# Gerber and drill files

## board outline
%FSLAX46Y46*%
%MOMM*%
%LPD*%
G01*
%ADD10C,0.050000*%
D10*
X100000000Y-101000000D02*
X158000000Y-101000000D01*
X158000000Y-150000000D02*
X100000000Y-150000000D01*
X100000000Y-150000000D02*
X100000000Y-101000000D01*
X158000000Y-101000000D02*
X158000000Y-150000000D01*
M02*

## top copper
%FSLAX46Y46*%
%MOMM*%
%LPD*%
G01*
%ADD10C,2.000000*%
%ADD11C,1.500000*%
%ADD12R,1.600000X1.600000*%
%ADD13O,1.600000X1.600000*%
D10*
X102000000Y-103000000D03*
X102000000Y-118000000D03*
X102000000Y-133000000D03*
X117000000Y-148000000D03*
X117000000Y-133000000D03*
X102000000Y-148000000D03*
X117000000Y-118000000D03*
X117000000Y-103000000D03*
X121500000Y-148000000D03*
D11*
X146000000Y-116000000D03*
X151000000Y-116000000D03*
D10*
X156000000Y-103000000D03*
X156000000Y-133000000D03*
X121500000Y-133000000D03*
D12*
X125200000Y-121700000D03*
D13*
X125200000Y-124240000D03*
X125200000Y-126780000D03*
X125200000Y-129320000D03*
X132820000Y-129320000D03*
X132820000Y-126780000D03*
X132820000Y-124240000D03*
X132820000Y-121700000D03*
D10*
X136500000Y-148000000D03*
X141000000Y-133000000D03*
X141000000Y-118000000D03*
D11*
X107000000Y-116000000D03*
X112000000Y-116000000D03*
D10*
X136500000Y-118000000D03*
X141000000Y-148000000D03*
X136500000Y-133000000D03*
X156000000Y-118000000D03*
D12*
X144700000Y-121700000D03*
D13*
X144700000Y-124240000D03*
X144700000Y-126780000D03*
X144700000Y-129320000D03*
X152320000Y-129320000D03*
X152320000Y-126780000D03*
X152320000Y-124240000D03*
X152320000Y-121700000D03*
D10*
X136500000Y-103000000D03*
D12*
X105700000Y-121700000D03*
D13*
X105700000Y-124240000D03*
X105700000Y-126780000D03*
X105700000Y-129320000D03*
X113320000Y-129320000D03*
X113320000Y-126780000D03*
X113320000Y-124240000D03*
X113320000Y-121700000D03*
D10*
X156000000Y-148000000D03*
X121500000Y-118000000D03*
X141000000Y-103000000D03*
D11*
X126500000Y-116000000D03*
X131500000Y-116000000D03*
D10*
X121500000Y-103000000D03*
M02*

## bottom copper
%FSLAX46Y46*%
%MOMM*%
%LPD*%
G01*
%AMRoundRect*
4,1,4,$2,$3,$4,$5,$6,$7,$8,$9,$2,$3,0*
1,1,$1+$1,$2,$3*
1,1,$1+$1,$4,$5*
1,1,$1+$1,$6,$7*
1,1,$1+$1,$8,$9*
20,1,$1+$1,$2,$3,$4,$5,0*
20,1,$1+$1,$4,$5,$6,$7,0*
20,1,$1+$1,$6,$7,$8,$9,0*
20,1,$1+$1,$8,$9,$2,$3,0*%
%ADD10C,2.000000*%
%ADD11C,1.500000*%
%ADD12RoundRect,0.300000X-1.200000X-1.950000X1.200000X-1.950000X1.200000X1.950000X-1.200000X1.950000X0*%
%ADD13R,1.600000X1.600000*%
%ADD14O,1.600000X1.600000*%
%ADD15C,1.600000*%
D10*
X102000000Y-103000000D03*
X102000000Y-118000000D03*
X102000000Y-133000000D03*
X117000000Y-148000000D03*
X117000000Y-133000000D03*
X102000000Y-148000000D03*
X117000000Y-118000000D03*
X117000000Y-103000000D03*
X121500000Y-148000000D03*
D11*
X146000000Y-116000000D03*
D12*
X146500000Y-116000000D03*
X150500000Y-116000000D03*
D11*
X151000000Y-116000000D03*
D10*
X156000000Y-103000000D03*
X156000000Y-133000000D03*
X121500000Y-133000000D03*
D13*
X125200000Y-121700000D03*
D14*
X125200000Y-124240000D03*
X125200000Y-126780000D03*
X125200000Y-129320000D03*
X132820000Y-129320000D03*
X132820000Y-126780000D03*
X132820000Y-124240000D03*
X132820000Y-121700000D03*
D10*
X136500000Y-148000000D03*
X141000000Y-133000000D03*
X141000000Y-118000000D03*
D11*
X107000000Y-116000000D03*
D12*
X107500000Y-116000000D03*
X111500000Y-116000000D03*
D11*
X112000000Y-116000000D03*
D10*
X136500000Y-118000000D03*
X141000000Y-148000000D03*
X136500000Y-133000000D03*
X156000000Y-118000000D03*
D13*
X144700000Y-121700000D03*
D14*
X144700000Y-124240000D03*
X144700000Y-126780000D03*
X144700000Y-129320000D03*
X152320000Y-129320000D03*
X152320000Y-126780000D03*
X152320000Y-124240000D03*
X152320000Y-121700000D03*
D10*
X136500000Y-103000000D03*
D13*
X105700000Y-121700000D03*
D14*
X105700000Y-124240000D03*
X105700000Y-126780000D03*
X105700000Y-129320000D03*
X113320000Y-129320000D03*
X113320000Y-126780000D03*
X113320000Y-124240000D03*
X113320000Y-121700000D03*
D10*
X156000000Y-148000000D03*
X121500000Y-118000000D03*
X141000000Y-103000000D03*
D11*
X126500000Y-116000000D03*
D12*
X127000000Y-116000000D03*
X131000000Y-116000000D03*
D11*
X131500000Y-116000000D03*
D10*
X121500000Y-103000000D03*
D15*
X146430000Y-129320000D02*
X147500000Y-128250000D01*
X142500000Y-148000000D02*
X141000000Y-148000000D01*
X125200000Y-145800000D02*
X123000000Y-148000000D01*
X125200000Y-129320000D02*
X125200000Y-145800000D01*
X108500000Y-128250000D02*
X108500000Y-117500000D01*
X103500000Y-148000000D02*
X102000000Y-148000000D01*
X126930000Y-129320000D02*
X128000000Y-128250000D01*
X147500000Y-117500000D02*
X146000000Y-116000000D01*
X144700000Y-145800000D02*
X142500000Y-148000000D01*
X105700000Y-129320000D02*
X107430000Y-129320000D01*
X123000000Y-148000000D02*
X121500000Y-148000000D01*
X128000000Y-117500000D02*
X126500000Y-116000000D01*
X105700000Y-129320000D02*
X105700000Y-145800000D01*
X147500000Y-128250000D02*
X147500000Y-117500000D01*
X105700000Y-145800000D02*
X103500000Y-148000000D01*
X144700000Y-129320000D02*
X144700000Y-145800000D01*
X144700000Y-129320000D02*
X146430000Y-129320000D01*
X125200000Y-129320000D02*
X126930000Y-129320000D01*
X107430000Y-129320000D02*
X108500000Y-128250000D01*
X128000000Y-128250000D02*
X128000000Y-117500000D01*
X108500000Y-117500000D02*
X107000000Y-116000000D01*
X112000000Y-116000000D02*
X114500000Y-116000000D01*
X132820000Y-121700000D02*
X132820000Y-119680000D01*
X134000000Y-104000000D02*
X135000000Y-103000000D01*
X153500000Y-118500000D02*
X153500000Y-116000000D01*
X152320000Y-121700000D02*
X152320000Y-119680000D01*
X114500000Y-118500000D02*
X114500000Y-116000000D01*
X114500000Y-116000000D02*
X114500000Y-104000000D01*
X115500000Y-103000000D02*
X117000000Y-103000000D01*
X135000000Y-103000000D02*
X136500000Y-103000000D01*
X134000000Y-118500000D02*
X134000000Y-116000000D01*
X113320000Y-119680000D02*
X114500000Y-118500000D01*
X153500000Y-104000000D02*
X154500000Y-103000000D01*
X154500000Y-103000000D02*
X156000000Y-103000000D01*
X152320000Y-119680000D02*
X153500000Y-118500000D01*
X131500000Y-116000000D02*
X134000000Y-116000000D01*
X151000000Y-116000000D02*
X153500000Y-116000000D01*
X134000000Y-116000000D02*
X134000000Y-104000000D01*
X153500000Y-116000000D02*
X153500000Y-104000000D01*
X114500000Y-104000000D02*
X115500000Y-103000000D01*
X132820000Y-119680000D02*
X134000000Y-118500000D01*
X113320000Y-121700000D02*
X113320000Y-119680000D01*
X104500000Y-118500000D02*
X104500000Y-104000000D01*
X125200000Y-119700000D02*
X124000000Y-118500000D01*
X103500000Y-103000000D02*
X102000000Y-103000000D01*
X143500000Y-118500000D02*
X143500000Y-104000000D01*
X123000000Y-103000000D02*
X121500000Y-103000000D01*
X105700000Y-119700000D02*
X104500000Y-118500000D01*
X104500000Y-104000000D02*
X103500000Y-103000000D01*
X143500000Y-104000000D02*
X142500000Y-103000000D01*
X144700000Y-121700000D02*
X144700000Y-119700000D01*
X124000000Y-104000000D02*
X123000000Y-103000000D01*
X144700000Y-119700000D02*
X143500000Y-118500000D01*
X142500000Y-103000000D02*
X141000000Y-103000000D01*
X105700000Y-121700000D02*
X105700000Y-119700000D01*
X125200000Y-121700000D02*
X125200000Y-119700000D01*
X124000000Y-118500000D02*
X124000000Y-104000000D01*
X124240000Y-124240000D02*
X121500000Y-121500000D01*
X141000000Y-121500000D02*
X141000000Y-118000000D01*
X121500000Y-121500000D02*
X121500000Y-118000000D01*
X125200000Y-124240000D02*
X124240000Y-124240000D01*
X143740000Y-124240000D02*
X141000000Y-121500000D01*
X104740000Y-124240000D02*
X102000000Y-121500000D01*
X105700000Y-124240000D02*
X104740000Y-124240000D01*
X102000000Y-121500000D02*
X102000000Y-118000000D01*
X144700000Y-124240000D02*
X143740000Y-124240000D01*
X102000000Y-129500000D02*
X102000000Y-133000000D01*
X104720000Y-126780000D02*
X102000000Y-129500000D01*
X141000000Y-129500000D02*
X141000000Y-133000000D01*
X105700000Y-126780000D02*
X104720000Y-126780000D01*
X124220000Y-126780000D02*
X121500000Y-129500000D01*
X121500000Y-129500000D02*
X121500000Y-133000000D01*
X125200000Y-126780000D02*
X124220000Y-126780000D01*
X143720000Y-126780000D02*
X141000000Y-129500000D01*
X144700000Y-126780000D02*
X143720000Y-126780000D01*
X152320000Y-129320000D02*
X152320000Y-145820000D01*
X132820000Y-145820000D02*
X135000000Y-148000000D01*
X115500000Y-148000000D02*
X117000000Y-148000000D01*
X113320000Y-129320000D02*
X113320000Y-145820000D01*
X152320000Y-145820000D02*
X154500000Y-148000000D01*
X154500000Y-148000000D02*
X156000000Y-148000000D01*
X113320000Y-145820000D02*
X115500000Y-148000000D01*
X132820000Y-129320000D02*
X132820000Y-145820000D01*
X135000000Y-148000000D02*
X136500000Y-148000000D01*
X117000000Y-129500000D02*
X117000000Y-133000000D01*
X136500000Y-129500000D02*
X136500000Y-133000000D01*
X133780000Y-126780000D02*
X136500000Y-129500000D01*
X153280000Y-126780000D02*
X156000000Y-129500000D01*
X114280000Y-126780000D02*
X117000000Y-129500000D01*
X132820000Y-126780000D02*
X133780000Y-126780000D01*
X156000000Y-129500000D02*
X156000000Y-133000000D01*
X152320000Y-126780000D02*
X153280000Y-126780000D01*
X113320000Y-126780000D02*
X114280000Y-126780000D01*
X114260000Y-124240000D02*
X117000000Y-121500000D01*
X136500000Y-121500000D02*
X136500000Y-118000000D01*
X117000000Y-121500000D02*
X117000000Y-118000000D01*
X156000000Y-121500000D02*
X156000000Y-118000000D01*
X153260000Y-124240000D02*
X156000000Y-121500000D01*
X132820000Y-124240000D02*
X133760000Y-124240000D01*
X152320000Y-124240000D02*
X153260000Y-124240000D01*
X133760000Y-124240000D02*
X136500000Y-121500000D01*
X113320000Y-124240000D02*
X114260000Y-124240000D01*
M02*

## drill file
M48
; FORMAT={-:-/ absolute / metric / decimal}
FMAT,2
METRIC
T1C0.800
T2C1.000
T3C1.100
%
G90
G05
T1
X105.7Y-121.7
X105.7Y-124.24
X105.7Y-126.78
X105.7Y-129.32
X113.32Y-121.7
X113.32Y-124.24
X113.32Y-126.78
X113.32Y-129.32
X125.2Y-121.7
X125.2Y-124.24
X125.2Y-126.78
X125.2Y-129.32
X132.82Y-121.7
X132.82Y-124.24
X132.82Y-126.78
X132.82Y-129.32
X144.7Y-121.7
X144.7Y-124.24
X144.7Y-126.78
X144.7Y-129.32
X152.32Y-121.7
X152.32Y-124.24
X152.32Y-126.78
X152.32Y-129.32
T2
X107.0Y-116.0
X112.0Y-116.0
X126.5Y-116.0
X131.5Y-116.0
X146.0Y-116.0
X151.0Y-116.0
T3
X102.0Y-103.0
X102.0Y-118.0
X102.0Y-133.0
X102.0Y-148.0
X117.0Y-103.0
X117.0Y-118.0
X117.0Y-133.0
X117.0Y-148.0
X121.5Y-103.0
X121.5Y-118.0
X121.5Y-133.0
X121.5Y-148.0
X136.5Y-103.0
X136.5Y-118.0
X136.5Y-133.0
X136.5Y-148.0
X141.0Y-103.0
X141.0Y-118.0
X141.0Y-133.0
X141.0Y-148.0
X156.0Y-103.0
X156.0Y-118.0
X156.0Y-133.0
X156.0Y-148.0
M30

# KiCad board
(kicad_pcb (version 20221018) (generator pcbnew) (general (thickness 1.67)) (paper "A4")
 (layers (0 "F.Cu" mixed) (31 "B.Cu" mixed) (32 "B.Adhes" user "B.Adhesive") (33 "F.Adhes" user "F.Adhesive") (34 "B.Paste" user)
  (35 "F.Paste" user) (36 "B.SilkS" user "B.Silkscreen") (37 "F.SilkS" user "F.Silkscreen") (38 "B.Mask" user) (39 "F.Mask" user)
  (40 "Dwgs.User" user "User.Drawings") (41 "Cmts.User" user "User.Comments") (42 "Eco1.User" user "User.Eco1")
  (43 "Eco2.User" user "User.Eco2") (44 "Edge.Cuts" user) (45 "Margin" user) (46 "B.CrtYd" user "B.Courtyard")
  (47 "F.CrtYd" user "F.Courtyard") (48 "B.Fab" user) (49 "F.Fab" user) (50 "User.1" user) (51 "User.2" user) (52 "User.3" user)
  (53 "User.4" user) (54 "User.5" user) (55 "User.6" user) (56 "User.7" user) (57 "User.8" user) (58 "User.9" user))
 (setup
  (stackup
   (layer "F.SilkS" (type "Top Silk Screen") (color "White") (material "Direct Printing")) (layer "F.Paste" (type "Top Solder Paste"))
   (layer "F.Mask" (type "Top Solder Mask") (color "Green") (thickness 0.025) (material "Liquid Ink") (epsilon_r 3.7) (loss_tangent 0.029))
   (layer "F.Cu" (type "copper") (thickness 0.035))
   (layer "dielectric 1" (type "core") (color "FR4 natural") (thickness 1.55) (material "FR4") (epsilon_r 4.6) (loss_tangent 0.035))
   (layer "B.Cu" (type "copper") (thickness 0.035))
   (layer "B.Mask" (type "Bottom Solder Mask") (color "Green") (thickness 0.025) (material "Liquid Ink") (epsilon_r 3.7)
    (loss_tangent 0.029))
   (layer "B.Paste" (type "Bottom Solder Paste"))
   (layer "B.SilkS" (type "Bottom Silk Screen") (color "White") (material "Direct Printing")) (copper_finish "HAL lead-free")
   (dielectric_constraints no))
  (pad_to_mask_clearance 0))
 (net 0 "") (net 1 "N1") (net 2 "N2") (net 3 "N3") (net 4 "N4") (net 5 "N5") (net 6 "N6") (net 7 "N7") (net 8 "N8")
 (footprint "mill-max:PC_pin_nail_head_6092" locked (layer "F.Cu") (at 102 103)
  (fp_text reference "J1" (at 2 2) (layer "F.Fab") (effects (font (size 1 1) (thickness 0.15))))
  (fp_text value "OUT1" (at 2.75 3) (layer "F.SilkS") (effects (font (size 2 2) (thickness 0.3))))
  (pad "1" thru_hole circle locked (at 0 0) (size 2 2) (drill 1.1) (layers "*.Cu" "*.Mask") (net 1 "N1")))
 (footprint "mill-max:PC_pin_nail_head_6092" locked (layer "F.Cu") (at 102 118)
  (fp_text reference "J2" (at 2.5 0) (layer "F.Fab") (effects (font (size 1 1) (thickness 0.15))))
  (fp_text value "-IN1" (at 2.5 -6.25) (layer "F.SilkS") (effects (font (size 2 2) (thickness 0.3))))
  (pad "1" thru_hole circle locked (at 0 0) (size 2 2) (drill 1.1) (layers "*.Cu" "*.Mask") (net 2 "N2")))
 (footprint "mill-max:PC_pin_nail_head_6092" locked (layer "F.Cu") (at 102 133)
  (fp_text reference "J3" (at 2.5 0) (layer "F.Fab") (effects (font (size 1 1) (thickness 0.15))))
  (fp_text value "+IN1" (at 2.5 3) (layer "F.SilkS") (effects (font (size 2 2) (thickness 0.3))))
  (pad "1" thru_hole circle locked (at 0 0) (size 2 2) (drill 1.1) (layers "*.Cu" "*.Mask") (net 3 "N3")))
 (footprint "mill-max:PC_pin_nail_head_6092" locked (layer "F.Cu") (at 117 148)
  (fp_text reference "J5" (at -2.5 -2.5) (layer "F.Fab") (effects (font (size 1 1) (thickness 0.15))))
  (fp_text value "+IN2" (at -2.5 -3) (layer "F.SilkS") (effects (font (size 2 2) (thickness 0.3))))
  (pad "1" thru_hole circle locked (at 0 0) (size 2 2) (drill 1.1) (layers "*.Cu" "*.Mask") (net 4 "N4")))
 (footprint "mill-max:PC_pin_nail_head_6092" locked (layer "F.Cu") (at 117 133)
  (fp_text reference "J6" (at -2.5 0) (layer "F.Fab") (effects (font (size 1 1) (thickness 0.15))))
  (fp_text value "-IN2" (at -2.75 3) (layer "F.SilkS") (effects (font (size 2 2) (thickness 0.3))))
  (pad "1" thru_hole circle locked (at 0 0) (size 2 2) (drill 1.1) (layers "*.Cu" "*.Mask") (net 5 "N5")))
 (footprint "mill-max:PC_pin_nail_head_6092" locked (layer "F.Cu") (at 102 148)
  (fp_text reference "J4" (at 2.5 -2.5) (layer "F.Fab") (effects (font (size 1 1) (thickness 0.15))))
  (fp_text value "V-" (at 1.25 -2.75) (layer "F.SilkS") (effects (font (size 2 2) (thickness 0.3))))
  (pad "1" thru_hole circle locked (at 0 0) (size 2 2) (drill 1.1) (layers "*.Cu" "*.Mask") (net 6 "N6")))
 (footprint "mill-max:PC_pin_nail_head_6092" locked (layer "F.Cu") (at 117 118)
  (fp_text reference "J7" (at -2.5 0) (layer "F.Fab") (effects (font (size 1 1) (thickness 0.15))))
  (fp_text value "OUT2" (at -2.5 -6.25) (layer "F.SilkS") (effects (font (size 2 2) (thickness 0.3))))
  (pad "1" thru_hole circle locked (at 0 0) (size 2 2) (drill 1.1) (layers "*.Cu" "*.Mask") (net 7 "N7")))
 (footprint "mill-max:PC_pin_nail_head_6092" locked (layer "F.Cu") (at 117 103)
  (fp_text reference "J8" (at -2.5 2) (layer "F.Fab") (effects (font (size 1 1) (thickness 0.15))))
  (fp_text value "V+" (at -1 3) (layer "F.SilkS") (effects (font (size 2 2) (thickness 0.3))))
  (pad "1" thru_hole circle locked (at 0 0) (size 2 2) (drill 1.1) (layers "*.Cu" "*.Mask") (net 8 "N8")))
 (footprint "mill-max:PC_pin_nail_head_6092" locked (layer "F.Cu") (at 121.5 148)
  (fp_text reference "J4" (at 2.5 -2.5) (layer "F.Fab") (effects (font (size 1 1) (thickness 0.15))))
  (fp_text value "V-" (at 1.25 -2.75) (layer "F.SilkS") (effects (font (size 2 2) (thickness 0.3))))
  (pad "1" thru_hole circle locked (at 0 0) (size 2 2) (drill 1.1) (layers "*.Cu" "*.Mask") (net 6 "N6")))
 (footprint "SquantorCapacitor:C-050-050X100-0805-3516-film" (layer "F.Cu") (at 148.5 116)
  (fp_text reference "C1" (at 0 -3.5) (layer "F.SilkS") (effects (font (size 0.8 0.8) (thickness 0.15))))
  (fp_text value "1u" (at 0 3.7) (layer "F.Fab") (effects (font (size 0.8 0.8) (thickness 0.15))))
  (pad "1" thru_hole circle (at -2.5 0) (size 1.5 1.5) (drill 1) (layers "*.Cu" "*.Mask") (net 6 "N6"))
  (pad "1" smd roundrect (at -2 0) (size 3 4.5) (layers "B.Cu" "B.Paste" "B.Mask") (roundrect_rratio 0.1) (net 6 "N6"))
  (pad "2" smd roundrect (at 2 0) (size 3 4.5) (layers "B.Cu" "B.Paste" "B.Mask") (roundrect_rratio 0.1) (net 8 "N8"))
  (pad "2" thru_hole circle (at 2.5 0) (size 1.5 1.5) (drill 1) (layers "*.Cu" "*.Mask") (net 8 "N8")))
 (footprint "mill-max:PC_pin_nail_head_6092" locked (layer "F.Cu") (at 156 103)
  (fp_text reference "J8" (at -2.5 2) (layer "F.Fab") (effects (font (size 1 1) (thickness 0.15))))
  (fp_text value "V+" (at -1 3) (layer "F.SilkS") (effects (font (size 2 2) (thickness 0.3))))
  (pad "1" thru_hole circle locked (at 0 0) (size 2 2) (drill 1.1) (layers "*.Cu" "*.Mask") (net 8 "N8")))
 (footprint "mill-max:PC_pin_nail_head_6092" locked (layer "F.Cu") (at 156 133)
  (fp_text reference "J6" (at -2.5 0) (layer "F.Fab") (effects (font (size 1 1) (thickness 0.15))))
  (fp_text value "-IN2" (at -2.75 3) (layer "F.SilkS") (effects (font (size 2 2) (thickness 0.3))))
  (pad "1" thru_hole circle locked (at 0 0) (size 2 2) (drill 1.1) (layers "*.Cu" "*.Mask") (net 5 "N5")))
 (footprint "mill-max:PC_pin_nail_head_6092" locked (layer "F.Cu") (at 121.5 133)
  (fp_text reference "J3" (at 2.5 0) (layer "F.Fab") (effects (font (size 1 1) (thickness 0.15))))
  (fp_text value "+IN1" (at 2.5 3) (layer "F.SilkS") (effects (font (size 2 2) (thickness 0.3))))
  (pad "1" thru_hole circle locked (at 0 0) (size 2 2) (drill 1.1) (layers "*.Cu" "*.Mask") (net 3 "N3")))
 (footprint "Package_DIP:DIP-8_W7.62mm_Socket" (layer "F.Cu") (at 125.2 121.7)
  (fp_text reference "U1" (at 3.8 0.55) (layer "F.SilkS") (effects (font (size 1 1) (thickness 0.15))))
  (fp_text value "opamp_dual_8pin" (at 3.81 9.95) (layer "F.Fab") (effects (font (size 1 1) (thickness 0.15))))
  (pad "1" thru_hole rect (at 0 0) (size 1.6 1.6) (drill 0.8) (layers "*.Cu" "*.Mask") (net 1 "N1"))
  (pad "2" thru_hole oval (at 0 2.54) (size 1.6 1.6) (drill 0.8) (layers "*.Cu" "*.Mask") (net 2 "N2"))
  (pad "3" thru_hole oval (at 0 5.08) (size 1.6 1.6) (drill 0.8) (layers "*.Cu" "*.Mask") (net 3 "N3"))
  (pad "4" thru_hole oval (at 0 7.62) (size 1.6 1.6) (drill 0.8) (layers "*.Cu" "*.Mask") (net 6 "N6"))
  (pad "5" thru_hole oval (at 7.62 7.62) (size 1.6 1.6) (drill 0.8) (layers "*.Cu" "*.Mask") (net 4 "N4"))
  (pad "6" thru_hole oval (at 7.62 5.08) (size 1.6 1.6) (drill 0.8) (layers "*.Cu" "*.Mask") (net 5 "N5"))
  (pad "7" thru_hole oval (at 7.62 2.54) (size 1.6 1.6) (drill 0.8) (layers "*.Cu" "*.Mask") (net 7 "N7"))
  (pad "8" thru_hole oval (at 7.62 0) (size 1.6 1.6) (drill 0.8) (layers "*.Cu" "*.Mask") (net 8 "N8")))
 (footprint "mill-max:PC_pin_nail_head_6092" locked (layer "F.Cu") (at 136.5 148)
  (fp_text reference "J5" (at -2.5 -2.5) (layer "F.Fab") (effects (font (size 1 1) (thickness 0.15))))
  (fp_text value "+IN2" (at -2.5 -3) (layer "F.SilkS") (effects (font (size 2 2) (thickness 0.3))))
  (pad "1" thru_hole circle locked (at 0 0) (size 2 2) (drill 1.1) (layers "*.Cu" "*.Mask") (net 4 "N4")))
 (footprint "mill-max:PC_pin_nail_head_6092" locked (layer "F.Cu") (at 141 133)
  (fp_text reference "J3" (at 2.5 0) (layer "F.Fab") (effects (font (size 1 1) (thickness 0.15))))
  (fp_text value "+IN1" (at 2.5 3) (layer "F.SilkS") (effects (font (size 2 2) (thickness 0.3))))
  (pad "1" thru_hole circle locked (at 0 0) (size 2 2) (drill 1.1) (layers "*.Cu" "*.Mask") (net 3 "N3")))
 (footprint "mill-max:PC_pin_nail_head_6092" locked (layer "F.Cu") (at 141 118)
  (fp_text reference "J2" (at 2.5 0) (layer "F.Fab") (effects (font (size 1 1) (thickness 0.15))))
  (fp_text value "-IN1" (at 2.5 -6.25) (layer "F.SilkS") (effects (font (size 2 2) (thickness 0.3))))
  (pad "1" thru_hole circle locked (at 0 0) (size 2 2) (drill 1.1) (layers "*.Cu" "*.Mask") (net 2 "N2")))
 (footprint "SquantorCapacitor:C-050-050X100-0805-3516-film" (layer "F.Cu") (at 109.5 116)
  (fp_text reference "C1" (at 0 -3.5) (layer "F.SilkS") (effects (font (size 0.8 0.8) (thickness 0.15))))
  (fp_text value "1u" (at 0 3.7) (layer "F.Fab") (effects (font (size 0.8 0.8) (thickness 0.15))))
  (pad "1" thru_hole circle (at -2.5 0) (size 1.5 1.5) (drill 1) (layers "*.Cu" "*.Mask") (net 6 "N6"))
  (pad "1" smd roundrect (at -2 0) (size 3 4.5) (layers "B.Cu" "B.Paste" "B.Mask") (roundrect_rratio 0.1) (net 6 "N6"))
  (pad "2" smd roundrect (at 2 0) (size 3 4.5) (layers "B.Cu" "B.Paste" "B.Mask") (roundrect_rratio 0.1) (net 8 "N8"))
  (pad "2" thru_hole circle (at 2.5 0) (size 1.5 1.5) (drill 1) (layers "*.Cu" "*.Mask") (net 8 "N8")))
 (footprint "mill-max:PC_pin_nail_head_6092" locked (layer "F.Cu") (at 136.5 118)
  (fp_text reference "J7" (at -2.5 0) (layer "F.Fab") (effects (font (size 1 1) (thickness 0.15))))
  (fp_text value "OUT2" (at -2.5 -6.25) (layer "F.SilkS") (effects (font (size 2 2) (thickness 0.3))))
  (pad "1" thru_hole circle locked (at 0 0) (size 2 2) (drill 1.1) (layers "*.Cu" "*.Mask") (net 7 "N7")))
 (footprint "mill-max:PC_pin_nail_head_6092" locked (layer "F.Cu") (at 141 148)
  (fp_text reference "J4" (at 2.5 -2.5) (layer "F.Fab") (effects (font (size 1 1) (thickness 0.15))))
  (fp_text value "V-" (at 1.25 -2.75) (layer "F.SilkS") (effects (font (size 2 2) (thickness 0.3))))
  (pad "1" thru_hole circle locked (at 0 0) (size 2 2) (drill 1.1) (layers "*.Cu" "*.Mask") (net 6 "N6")))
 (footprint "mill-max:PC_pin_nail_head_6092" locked (layer "F.Cu") (at 136.5 133)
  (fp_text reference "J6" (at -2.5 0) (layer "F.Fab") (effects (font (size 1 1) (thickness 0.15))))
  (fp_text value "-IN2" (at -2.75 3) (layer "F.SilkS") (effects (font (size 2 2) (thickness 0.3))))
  (pad "1" thru_hole circle locked (at 0 0) (size 2 2) (drill 1.1) (layers "*.Cu" "*.Mask") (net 5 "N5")))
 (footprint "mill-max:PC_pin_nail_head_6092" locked (layer "F.Cu") (at 156 118)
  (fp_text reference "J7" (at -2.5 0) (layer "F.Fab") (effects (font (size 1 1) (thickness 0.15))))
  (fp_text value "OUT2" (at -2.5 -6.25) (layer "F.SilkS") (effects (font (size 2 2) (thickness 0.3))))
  (pad "1" thru_hole circle locked (at 0 0) (size 2 2) (drill 1.1) (layers "*.Cu" "*.Mask") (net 7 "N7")))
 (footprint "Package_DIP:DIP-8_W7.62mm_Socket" (layer "F.Cu") (at 144.7 121.7)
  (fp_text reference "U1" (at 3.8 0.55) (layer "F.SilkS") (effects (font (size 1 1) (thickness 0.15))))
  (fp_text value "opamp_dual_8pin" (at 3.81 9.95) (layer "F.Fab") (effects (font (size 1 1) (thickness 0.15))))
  (pad "1" thru_hole rect (at 0 0) (size 1.6 1.6) (drill 0.8) (layers "*.Cu" "*.Mask") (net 1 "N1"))
  (pad "2" thru_hole oval (at 0 2.54) (size 1.6 1.6) (drill 0.8) (layers "*.Cu" "*.Mask") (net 2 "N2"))
  (pad "3" thru_hole oval (at 0 5.08) (size 1.6 1.6) (drill 0.8) (layers "*.Cu" "*.Mask") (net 3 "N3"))
  (pad "4" thru_hole oval (at 0 7.62) (size 1.6 1.6) (drill 0.8) (layers "*.Cu" "*.Mask") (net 6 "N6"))
  (pad "5" thru_hole oval (at 7.62 7.62) (size 1.6 1.6) (drill 0.8) (layers "*.Cu" "*.Mask") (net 4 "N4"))
  (pad "6" thru_hole oval (at 7.62 5.08) (size 1.6 1.6) (drill 0.8) (layers "*.Cu" "*.Mask") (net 5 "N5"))
  (pad "7" thru_hole oval (at 7.62 2.54) (size 1.6 1.6) (drill 0.8) (layers "*.Cu" "*.Mask") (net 7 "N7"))
  (pad "8" thru_hole oval (at 7.62 0) (size 1.6 1.6) (drill 0.8) (layers "*.Cu" "*.Mask") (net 8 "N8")))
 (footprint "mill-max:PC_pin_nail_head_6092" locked (layer "F.Cu") (at 136.5 103)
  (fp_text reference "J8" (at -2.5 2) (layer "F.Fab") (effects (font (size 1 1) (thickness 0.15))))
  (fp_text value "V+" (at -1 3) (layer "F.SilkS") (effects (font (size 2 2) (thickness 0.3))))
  (pad "1" thru_hole circle locked (at 0 0) (size 2 2) (drill 1.1) (layers "*.Cu" "*.Mask") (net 8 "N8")))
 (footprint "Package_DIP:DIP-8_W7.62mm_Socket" (layer "F.Cu") (at 105.7 121.7)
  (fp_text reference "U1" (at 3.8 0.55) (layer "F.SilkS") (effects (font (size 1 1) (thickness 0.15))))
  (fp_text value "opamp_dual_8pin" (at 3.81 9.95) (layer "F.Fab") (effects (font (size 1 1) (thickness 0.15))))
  (pad "1" thru_hole rect (at 0 0) (size 1.6 1.6) (drill 0.8) (layers "*.Cu" "*.Mask") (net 1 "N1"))
  (pad "2" thru_hole oval (at 0 2.54) (size 1.6 1.6) (drill 0.8) (layers "*.Cu" "*.Mask") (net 2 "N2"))
  (pad "3" thru_hole oval (at 0 5.08) (size 1.6 1.6) (drill 0.8) (layers "*.Cu" "*.Mask") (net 3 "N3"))
  (pad "4" thru_hole oval (at 0 7.62) (size 1.6 1.6) (drill 0.8) (layers "*.Cu" "*.Mask") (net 6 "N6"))
  (pad "5" thru_hole oval (at 7.62 7.62) (size 1.6 1.6) (drill 0.8) (layers "*.Cu" "*.Mask") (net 4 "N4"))
  (pad "6" thru_hole oval (at 7.62 5.08) (size 1.6 1.6) (drill 0.8) (layers "*.Cu" "*.Mask") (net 5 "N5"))
  (pad "7" thru_hole oval (at 7.62 2.54) (size 1.6 1.6) (drill 0.8) (layers "*.Cu" "*.Mask") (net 7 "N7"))
  (pad "8" thru_hole oval (at 7.62 0) (size 1.6 1.6) (drill 0.8) (layers "*.Cu" "*.Mask") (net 8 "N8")))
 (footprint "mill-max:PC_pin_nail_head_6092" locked (layer "F.Cu") (at 156 148)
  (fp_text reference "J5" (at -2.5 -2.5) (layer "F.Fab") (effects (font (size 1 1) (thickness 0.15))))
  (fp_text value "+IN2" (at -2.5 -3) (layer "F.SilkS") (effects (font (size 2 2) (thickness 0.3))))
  (pad "1" thru_hole circle locked (at 0 0) (size 2 2) (drill 1.1) (layers "*.Cu" "*.Mask") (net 4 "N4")))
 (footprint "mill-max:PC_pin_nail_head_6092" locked (layer "F.Cu") (at 121.5 118)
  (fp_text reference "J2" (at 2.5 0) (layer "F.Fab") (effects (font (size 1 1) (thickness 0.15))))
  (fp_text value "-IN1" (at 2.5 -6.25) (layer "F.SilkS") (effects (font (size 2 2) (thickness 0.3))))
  (pad "1" thru_hole circle locked (at 0 0) (size 2 2) (drill 1.1) (layers "*.Cu" "*.Mask") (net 2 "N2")))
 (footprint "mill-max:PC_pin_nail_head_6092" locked (layer "F.Cu") (at 141 103)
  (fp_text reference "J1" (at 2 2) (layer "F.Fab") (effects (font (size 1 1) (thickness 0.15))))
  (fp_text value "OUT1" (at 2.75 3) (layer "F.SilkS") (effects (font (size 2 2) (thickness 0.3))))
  (pad "1" thru_hole circle locked (at 0 0) (size 2 2) (drill 1.1) (layers "*.Cu" "*.Mask") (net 1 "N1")))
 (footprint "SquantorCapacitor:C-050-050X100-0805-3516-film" (layer "F.Cu") (at 129 116)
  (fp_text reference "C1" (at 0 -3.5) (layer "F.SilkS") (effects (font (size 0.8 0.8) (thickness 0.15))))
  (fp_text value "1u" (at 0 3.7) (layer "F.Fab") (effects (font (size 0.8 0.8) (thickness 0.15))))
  (pad "1" thru_hole circle (at -2.5 0) (size 1.5 1.5) (drill 1) (layers "*.Cu" "*.Mask") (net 6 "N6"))
  (pad "1" smd roundrect (at -2 0) (size 3 4.5) (layers "B.Cu" "B.Paste" "B.Mask") (roundrect_rratio 0.1) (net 6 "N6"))
  (pad "2" smd roundrect (at 2 0) (size 3 4.5) (layers "B.Cu" "B.Paste" "B.Mask") (roundrect_rratio 0.1) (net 8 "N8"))
  (pad "2" thru_hole circle (at 2.5 0) (size 1.5 1.5) (drill 1) (layers "*.Cu" "*.Mask") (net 8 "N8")))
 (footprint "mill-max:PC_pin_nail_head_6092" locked (layer "F.Cu") (at 121.5 103)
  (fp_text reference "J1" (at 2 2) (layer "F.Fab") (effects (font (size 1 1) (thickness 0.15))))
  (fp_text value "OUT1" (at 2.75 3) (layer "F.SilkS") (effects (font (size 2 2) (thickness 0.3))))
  (pad "1" thru_hole circle locked (at 0 0) (size 2 2) (drill 1.1) (layers "*.Cu" "*.Mask") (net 1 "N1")))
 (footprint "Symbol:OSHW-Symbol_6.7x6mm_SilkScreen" (layer "B.Cu") (at 109 145 180)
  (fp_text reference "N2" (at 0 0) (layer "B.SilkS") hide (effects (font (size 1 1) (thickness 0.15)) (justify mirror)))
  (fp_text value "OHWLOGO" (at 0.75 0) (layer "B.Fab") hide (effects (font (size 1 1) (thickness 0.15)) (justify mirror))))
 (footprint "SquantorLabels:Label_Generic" (layer "B.Cu") (at 108 149)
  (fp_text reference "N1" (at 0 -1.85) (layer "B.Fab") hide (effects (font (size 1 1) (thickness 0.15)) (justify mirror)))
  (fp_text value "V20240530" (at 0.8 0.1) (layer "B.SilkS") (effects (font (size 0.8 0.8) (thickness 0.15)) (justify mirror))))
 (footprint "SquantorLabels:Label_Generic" (layer "B.Cu") (at 127.5 149)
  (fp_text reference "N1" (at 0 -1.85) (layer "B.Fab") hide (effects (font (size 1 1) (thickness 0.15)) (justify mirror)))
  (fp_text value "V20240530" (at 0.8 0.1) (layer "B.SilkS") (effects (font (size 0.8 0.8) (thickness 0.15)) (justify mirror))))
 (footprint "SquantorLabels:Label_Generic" (layer "B.Cu") (at 147 149)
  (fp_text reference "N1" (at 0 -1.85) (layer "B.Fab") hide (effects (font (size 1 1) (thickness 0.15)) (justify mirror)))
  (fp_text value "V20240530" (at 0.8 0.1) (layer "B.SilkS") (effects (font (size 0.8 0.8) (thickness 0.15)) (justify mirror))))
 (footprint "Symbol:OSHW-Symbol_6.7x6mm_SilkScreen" (layer "B.Cu") (at 148 145 180)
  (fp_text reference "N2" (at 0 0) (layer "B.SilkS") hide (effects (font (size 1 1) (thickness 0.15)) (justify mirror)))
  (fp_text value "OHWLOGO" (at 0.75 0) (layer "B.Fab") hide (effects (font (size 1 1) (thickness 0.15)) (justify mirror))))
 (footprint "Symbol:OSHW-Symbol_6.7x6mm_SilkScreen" (layer "B.Cu") (at 128.5 145 180)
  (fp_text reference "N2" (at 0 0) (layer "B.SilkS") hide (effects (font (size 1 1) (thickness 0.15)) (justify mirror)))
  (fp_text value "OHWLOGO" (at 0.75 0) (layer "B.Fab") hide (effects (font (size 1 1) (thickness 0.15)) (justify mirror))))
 (gr_line (start 100 101) (end 158 101) (stroke (width 0.05) (type default)) (layer "Edge.Cuts"))
 (gr_line (start 158 150) (end 100 150) (stroke (width 0.05) (type default)) (layer "Edge.Cuts"))
 (gr_line (start 100 150) (end 100 101) (stroke (width 0.05) (type default)) (layer "Edge.Cuts"))
 (gr_line (start 158 101) (end 158 150) (stroke (width 0.05) (type default)) (layer "Edge.Cuts"))
 (segment (start 146.43 129.32) (end 147.5 128.25) (width 1.6) (layer "B.Cu") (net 6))
 (segment (start 142.5 148) (end 141 148) (width 1.6) (layer "B.Cu") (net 6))
 (segment (start 125.2 145.8) (end 123 148) (width 1.6) (layer "B.Cu") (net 6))
 (segment (start 125.2 129.32) (end 125.2 145.8) (width 1.6) (layer "B.Cu") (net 6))
 (segment (start 108.5 128.25) (end 108.5 117.5) (width 1.6) (layer "B.Cu") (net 6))
 (segment (start 103.5 148) (end 102 148) (width 1.6) (layer "B.Cu") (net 6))
 (segment (start 126.93 129.32) (end 128 128.25) (width 1.6) (layer "B.Cu") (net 6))
 (segment (start 147.5 117.5) (end 146 116) (width 1.6) (layer "B.Cu") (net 6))
 (segment (start 144.7 145.8) (end 142.5 148) (width 1.6) (layer "B.Cu") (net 6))
 (segment (start 105.7 129.32) (end 107.43 129.32) (width 1.6) (layer "B.Cu") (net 6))
 (segment (start 123 148) (end 121.5 148) (width 1.6) (layer "B.Cu") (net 6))
 (segment (start 128 117.5) (end 126.5 116) (width 1.6) (layer "B.Cu") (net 6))
 (segment (start 105.7 129.32) (end 105.7 145.8) (width 1.6) (layer "B.Cu") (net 6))
 (segment (start 147.5 128.25) (end 147.5 117.5) (width 1.6) (layer "B.Cu") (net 6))
 (segment (start 105.7 145.8) (end 103.5 148) (width 1.6) (layer "B.Cu") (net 6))
 (segment (start 144.7 129.32) (end 144.7 145.8) (width 1.6) (layer "B.Cu") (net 6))
 (segment (start 144.7 129.32) (end 146.43 129.32) (width 1.6) (layer "B.Cu") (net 6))
 (segment (start 125.2 129.32) (end 126.93 129.32) (width 1.6) (layer "B.Cu") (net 6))
 (segment (start 107.43 129.32) (end 108.5 128.25) (width 1.6) (layer "B.Cu") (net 6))
 (segment (start 128 128.25) (end 128 117.5) (width 1.6) (layer "B.Cu") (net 6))
 (segment (start 108.5 117.5) (end 107 116) (width 1.6) (layer "B.Cu") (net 6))
 (segment (start 112 116) (end 114.5 116) (width 1.6) (layer "B.Cu") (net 8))
 (segment (start 132.82 121.7) (end 132.82 119.68) (width 1.6) (layer "B.Cu") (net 8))
 (segment (start 134 104) (end 135 103) (width 1.6) (layer "B.Cu") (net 8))
 (segment (start 153.5 118.5) (end 153.5 116) (width 1.6) (layer "B.Cu") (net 8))
 (segment (start 152.32 121.7) (end 152.32 119.68) (width 1.6) (layer "B.Cu") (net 8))
 (segment (start 114.5 118.5) (end 114.5 116) (width 1.6) (layer "B.Cu") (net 8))
 (segment (start 114.5 116) (end 114.5 104) (width 1.6) (layer "B.Cu") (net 8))
 (segment (start 115.5 103) (end 117 103) (width 1.6) (layer "B.Cu") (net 8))
 (segment (start 135 103) (end 136.5 103) (width 1.6) (layer "B.Cu") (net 8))
 (segment (start 134 118.5) (end 134 116) (width 1.6) (layer "B.Cu") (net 8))
 (segment (start 113.32 119.68) (end 114.5 118.5) (width 1.6) (layer "B.Cu") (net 8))
 (segment (start 153.5 104) (end 154.5 103) (width 1.6) (layer "B.Cu") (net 8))
 (segment (start 154.5 103) (end 156 103) (width 1.6) (layer "B.Cu") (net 8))
 (segment (start 152.32 119.68) (end 153.5 118.5) (width 1.6) (layer "B.Cu") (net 8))
 (segment (start 131.5 116) (end 134 116) (width 1.6) (layer "B.Cu") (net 8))
 (segment (start 151 116) (end 153.5 116) (width 1.6) (layer "B.Cu") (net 8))
 (segment (start 134 116) (end 134 104) (width 1.6) (layer "B.Cu") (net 8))
 (segment (start 153.5 116) (end 153.5 104) (width 1.6) (layer "B.Cu") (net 8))
 (segment (start 114.5 104) (end 115.5 103) (width 1.6) (layer "B.Cu") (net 8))
 (segment (start 132.82 119.68) (end 134 118.5) (width 1.6) (layer "B.Cu") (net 8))
 (segment (start 113.32 121.7) (end 113.32 119.68) (width 1.6) (layer "B.Cu") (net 8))
 (segment (start 104.5 118.5) (end 104.5 104) (width 1.6) (layer "B.Cu") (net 1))
 (segment (start 125.2 119.7) (end 124 118.5) (width 1.6) (layer "B.Cu") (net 1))
 (segment (start 103.5 103) (end 102 103) (width 1.6) (layer "B.Cu") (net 1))
 (segment (start 143.5 118.5) (end 143.5 104) (width 1.6) (layer "B.Cu") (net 1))
 (segment (start 123 103) (end 121.5 103) (width 1.6) (layer "B.Cu") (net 1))
 (segment (start 105.7 119.7) (end 104.5 118.5) (width 1.6) (layer "B.Cu") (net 1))
 (segment (start 104.5 104) (end 103.5 103) (width 1.6) (layer "B.Cu") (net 1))
 (segment (start 143.5 104) (end 142.5 103) (width 1.6) (layer "B.Cu") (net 1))
 (segment (start 144.7 121.7) (end 144.7 119.7) (width 1.6) (layer "B.Cu") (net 1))
 (segment (start 124 104) (end 123 103) (width 1.6) (layer "B.Cu") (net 1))
 (segment (start 144.7 119.7) (end 143.5 118.5) (width 1.6) (layer "B.Cu") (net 1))
 (segment (start 142.5 103) (end 141 103) (width 1.6) (layer "B.Cu") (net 1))
 (segment (start 105.7 121.7) (end 105.7 119.7) (width 1.6) (layer "B.Cu") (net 1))
 (segment (start 125.2 121.7) (end 125.2 119.7) (width 1.6) (layer "B.Cu") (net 1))
 (segment (start 124 118.5) (end 124 104) (width 1.6) (layer "B.Cu") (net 1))
 (segment (start 124.24 124.24) (end 121.5 121.5) (width 1.6) (layer "B.Cu") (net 2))
 (segment (start 141 121.5) (end 141 118) (width 1.6) (layer "B.Cu") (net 2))
 (segment (start 121.5 121.5) (end 121.5 118) (width 1.6) (layer "B.Cu") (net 2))
 (segment (start 125.2 124.24) (end 124.24 124.24) (width 1.6) (layer "B.Cu") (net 2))
 (segment (start 143.74 124.24) (end 141 121.5) (width 1.6) (layer "B.Cu") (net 2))
 (segment (start 104.74 124.24) (end 102 121.5) (width 1.6) (layer "B.Cu") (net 2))
 (segment (start 105.7 124.24) (end 104.74 124.24) (width 1.6) (layer "B.Cu") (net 2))
 (segment (start 102 121.5) (end 102 118) (width 1.6) (layer "B.Cu") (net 2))
 (segment (start 144.7 124.24) (end 143.74 124.24) (width 1.6) (layer "B.Cu") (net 2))
 (segment (start 102 129.5) (end 102 133) (width 1.6) (layer "B.Cu") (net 3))
 (segment (start 104.72 126.78) (end 102 129.5) (width 1.6) (layer "B.Cu") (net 3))
 (segment (start 141 129.5) (end 141 133) (width 1.6) (layer "B.Cu") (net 3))
 (segment (start 105.7 126.78) (end 104.72 126.78) (width 1.6) (layer "B.Cu") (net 3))
 (segment (start 124.22 126.78) (end 121.5 129.5) (width 1.6) (layer "B.Cu") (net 3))
 (segment (start 121.5 129.5) (end 121.5 133) (width 1.6) (layer "B.Cu") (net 3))
 (segment (start 125.2 126.78) (end 124.22 126.78) (width 1.6) (layer "B.Cu") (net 3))
 (segment (start 143.72 126.78) (end 141 129.5) (width 1.6) (layer "B.Cu") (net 3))
 (segment (start 144.7 126.78) (end 143.72 126.78) (width 1.6) (layer "B.Cu") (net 3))
 (segment (start 152.32 129.32) (end 152.32 145.82) (width 1.6) (layer "B.Cu") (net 4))
 (segment (start 132.82 145.82) (end 135 148) (width 1.6) (layer "B.Cu") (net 4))
 (segment (start 115.5 148) (end 117 148) (width 1.6) (layer "B.Cu") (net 4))
 (segment (start 113.32 129.32) (end 113.32 145.82) (width 1.6) (layer "B.Cu") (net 4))
 (segment (start 152.32 145.82) (end 154.5 148) (width 1.6) (layer "B.Cu") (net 4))
 (segment (start 154.5 148) (end 156 148) (width 1.6) (layer "B.Cu") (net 4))
 (segment (start 113.32 145.82) (end 115.5 148) (width 1.6) (layer "B.Cu") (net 4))
 (segment (start 132.82 129.32) (end 132.82 145.82) (width 1.6) (layer "B.Cu") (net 4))
 (segment (start 135 148) (end 136.5 148) (width 1.6) (layer "B.Cu") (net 4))
 (segment (start 117 129.5) (end 117 133) (width 1.6) (layer "B.Cu") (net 5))
 (segment (start 136.5 129.5) (end 136.5 133) (width 1.6) (layer "B.Cu") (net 5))
 (segment (start 133.78 126.78) (end 136.5 129.5) (width 1.6) (layer "B.Cu") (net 5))
 (segment (start 153.28 126.78) (end 156 129.5) (width 1.6) (layer "B.Cu") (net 5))
 (segment (start 114.28 126.78) (end 117 129.5) (width 1.6) (layer "B.Cu") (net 5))
 (segment (start 132.82 126.78) (end 133.78 126.78) (width 1.6) (layer "B.Cu") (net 5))
 (segment (start 156 129.5) (end 156 133) (width 1.6) (layer "B.Cu") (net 5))
 (segment (start 152.32 126.78) (end 153.28 126.78) (width 1.6) (layer "B.Cu") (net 5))
 (segment (start 113.32 126.78) (end 114.28 126.78) (width 1.6) (layer "B.Cu") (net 5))
 (segment (start 114.26 124.24) (end 117 121.5) (width 1.6) (layer "B.Cu") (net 7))
 (segment (start 136.5 121.5) (end 136.5 118) (width 1.6) (layer "B.Cu") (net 7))
 (segment (start 117 121.5) (end 117 118) (width 1.6) (layer "B.Cu") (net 7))
 (segment (start 156 121.5) (end 156 118) (width 1.6) (layer "B.Cu") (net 7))
 (segment (start 153.26 124.24) (end 156 121.5) (width 1.6) (layer "B.Cu") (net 7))
 (segment (start 132.82 124.24) (end 133.76 124.24) (width 1.6) (layer "B.Cu") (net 7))
 (segment (start 152.32 124.24) (end 153.26 124.24) (width 1.6) (layer "B.Cu") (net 7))
 (segment (start 133.76 124.24) (end 136.5 121.5) (width 1.6) (layer "B.Cu") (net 7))
 (segment (start 113.32 124.24) (end 114.26 124.24) (width 1.6) (layer "B.Cu") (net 7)))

